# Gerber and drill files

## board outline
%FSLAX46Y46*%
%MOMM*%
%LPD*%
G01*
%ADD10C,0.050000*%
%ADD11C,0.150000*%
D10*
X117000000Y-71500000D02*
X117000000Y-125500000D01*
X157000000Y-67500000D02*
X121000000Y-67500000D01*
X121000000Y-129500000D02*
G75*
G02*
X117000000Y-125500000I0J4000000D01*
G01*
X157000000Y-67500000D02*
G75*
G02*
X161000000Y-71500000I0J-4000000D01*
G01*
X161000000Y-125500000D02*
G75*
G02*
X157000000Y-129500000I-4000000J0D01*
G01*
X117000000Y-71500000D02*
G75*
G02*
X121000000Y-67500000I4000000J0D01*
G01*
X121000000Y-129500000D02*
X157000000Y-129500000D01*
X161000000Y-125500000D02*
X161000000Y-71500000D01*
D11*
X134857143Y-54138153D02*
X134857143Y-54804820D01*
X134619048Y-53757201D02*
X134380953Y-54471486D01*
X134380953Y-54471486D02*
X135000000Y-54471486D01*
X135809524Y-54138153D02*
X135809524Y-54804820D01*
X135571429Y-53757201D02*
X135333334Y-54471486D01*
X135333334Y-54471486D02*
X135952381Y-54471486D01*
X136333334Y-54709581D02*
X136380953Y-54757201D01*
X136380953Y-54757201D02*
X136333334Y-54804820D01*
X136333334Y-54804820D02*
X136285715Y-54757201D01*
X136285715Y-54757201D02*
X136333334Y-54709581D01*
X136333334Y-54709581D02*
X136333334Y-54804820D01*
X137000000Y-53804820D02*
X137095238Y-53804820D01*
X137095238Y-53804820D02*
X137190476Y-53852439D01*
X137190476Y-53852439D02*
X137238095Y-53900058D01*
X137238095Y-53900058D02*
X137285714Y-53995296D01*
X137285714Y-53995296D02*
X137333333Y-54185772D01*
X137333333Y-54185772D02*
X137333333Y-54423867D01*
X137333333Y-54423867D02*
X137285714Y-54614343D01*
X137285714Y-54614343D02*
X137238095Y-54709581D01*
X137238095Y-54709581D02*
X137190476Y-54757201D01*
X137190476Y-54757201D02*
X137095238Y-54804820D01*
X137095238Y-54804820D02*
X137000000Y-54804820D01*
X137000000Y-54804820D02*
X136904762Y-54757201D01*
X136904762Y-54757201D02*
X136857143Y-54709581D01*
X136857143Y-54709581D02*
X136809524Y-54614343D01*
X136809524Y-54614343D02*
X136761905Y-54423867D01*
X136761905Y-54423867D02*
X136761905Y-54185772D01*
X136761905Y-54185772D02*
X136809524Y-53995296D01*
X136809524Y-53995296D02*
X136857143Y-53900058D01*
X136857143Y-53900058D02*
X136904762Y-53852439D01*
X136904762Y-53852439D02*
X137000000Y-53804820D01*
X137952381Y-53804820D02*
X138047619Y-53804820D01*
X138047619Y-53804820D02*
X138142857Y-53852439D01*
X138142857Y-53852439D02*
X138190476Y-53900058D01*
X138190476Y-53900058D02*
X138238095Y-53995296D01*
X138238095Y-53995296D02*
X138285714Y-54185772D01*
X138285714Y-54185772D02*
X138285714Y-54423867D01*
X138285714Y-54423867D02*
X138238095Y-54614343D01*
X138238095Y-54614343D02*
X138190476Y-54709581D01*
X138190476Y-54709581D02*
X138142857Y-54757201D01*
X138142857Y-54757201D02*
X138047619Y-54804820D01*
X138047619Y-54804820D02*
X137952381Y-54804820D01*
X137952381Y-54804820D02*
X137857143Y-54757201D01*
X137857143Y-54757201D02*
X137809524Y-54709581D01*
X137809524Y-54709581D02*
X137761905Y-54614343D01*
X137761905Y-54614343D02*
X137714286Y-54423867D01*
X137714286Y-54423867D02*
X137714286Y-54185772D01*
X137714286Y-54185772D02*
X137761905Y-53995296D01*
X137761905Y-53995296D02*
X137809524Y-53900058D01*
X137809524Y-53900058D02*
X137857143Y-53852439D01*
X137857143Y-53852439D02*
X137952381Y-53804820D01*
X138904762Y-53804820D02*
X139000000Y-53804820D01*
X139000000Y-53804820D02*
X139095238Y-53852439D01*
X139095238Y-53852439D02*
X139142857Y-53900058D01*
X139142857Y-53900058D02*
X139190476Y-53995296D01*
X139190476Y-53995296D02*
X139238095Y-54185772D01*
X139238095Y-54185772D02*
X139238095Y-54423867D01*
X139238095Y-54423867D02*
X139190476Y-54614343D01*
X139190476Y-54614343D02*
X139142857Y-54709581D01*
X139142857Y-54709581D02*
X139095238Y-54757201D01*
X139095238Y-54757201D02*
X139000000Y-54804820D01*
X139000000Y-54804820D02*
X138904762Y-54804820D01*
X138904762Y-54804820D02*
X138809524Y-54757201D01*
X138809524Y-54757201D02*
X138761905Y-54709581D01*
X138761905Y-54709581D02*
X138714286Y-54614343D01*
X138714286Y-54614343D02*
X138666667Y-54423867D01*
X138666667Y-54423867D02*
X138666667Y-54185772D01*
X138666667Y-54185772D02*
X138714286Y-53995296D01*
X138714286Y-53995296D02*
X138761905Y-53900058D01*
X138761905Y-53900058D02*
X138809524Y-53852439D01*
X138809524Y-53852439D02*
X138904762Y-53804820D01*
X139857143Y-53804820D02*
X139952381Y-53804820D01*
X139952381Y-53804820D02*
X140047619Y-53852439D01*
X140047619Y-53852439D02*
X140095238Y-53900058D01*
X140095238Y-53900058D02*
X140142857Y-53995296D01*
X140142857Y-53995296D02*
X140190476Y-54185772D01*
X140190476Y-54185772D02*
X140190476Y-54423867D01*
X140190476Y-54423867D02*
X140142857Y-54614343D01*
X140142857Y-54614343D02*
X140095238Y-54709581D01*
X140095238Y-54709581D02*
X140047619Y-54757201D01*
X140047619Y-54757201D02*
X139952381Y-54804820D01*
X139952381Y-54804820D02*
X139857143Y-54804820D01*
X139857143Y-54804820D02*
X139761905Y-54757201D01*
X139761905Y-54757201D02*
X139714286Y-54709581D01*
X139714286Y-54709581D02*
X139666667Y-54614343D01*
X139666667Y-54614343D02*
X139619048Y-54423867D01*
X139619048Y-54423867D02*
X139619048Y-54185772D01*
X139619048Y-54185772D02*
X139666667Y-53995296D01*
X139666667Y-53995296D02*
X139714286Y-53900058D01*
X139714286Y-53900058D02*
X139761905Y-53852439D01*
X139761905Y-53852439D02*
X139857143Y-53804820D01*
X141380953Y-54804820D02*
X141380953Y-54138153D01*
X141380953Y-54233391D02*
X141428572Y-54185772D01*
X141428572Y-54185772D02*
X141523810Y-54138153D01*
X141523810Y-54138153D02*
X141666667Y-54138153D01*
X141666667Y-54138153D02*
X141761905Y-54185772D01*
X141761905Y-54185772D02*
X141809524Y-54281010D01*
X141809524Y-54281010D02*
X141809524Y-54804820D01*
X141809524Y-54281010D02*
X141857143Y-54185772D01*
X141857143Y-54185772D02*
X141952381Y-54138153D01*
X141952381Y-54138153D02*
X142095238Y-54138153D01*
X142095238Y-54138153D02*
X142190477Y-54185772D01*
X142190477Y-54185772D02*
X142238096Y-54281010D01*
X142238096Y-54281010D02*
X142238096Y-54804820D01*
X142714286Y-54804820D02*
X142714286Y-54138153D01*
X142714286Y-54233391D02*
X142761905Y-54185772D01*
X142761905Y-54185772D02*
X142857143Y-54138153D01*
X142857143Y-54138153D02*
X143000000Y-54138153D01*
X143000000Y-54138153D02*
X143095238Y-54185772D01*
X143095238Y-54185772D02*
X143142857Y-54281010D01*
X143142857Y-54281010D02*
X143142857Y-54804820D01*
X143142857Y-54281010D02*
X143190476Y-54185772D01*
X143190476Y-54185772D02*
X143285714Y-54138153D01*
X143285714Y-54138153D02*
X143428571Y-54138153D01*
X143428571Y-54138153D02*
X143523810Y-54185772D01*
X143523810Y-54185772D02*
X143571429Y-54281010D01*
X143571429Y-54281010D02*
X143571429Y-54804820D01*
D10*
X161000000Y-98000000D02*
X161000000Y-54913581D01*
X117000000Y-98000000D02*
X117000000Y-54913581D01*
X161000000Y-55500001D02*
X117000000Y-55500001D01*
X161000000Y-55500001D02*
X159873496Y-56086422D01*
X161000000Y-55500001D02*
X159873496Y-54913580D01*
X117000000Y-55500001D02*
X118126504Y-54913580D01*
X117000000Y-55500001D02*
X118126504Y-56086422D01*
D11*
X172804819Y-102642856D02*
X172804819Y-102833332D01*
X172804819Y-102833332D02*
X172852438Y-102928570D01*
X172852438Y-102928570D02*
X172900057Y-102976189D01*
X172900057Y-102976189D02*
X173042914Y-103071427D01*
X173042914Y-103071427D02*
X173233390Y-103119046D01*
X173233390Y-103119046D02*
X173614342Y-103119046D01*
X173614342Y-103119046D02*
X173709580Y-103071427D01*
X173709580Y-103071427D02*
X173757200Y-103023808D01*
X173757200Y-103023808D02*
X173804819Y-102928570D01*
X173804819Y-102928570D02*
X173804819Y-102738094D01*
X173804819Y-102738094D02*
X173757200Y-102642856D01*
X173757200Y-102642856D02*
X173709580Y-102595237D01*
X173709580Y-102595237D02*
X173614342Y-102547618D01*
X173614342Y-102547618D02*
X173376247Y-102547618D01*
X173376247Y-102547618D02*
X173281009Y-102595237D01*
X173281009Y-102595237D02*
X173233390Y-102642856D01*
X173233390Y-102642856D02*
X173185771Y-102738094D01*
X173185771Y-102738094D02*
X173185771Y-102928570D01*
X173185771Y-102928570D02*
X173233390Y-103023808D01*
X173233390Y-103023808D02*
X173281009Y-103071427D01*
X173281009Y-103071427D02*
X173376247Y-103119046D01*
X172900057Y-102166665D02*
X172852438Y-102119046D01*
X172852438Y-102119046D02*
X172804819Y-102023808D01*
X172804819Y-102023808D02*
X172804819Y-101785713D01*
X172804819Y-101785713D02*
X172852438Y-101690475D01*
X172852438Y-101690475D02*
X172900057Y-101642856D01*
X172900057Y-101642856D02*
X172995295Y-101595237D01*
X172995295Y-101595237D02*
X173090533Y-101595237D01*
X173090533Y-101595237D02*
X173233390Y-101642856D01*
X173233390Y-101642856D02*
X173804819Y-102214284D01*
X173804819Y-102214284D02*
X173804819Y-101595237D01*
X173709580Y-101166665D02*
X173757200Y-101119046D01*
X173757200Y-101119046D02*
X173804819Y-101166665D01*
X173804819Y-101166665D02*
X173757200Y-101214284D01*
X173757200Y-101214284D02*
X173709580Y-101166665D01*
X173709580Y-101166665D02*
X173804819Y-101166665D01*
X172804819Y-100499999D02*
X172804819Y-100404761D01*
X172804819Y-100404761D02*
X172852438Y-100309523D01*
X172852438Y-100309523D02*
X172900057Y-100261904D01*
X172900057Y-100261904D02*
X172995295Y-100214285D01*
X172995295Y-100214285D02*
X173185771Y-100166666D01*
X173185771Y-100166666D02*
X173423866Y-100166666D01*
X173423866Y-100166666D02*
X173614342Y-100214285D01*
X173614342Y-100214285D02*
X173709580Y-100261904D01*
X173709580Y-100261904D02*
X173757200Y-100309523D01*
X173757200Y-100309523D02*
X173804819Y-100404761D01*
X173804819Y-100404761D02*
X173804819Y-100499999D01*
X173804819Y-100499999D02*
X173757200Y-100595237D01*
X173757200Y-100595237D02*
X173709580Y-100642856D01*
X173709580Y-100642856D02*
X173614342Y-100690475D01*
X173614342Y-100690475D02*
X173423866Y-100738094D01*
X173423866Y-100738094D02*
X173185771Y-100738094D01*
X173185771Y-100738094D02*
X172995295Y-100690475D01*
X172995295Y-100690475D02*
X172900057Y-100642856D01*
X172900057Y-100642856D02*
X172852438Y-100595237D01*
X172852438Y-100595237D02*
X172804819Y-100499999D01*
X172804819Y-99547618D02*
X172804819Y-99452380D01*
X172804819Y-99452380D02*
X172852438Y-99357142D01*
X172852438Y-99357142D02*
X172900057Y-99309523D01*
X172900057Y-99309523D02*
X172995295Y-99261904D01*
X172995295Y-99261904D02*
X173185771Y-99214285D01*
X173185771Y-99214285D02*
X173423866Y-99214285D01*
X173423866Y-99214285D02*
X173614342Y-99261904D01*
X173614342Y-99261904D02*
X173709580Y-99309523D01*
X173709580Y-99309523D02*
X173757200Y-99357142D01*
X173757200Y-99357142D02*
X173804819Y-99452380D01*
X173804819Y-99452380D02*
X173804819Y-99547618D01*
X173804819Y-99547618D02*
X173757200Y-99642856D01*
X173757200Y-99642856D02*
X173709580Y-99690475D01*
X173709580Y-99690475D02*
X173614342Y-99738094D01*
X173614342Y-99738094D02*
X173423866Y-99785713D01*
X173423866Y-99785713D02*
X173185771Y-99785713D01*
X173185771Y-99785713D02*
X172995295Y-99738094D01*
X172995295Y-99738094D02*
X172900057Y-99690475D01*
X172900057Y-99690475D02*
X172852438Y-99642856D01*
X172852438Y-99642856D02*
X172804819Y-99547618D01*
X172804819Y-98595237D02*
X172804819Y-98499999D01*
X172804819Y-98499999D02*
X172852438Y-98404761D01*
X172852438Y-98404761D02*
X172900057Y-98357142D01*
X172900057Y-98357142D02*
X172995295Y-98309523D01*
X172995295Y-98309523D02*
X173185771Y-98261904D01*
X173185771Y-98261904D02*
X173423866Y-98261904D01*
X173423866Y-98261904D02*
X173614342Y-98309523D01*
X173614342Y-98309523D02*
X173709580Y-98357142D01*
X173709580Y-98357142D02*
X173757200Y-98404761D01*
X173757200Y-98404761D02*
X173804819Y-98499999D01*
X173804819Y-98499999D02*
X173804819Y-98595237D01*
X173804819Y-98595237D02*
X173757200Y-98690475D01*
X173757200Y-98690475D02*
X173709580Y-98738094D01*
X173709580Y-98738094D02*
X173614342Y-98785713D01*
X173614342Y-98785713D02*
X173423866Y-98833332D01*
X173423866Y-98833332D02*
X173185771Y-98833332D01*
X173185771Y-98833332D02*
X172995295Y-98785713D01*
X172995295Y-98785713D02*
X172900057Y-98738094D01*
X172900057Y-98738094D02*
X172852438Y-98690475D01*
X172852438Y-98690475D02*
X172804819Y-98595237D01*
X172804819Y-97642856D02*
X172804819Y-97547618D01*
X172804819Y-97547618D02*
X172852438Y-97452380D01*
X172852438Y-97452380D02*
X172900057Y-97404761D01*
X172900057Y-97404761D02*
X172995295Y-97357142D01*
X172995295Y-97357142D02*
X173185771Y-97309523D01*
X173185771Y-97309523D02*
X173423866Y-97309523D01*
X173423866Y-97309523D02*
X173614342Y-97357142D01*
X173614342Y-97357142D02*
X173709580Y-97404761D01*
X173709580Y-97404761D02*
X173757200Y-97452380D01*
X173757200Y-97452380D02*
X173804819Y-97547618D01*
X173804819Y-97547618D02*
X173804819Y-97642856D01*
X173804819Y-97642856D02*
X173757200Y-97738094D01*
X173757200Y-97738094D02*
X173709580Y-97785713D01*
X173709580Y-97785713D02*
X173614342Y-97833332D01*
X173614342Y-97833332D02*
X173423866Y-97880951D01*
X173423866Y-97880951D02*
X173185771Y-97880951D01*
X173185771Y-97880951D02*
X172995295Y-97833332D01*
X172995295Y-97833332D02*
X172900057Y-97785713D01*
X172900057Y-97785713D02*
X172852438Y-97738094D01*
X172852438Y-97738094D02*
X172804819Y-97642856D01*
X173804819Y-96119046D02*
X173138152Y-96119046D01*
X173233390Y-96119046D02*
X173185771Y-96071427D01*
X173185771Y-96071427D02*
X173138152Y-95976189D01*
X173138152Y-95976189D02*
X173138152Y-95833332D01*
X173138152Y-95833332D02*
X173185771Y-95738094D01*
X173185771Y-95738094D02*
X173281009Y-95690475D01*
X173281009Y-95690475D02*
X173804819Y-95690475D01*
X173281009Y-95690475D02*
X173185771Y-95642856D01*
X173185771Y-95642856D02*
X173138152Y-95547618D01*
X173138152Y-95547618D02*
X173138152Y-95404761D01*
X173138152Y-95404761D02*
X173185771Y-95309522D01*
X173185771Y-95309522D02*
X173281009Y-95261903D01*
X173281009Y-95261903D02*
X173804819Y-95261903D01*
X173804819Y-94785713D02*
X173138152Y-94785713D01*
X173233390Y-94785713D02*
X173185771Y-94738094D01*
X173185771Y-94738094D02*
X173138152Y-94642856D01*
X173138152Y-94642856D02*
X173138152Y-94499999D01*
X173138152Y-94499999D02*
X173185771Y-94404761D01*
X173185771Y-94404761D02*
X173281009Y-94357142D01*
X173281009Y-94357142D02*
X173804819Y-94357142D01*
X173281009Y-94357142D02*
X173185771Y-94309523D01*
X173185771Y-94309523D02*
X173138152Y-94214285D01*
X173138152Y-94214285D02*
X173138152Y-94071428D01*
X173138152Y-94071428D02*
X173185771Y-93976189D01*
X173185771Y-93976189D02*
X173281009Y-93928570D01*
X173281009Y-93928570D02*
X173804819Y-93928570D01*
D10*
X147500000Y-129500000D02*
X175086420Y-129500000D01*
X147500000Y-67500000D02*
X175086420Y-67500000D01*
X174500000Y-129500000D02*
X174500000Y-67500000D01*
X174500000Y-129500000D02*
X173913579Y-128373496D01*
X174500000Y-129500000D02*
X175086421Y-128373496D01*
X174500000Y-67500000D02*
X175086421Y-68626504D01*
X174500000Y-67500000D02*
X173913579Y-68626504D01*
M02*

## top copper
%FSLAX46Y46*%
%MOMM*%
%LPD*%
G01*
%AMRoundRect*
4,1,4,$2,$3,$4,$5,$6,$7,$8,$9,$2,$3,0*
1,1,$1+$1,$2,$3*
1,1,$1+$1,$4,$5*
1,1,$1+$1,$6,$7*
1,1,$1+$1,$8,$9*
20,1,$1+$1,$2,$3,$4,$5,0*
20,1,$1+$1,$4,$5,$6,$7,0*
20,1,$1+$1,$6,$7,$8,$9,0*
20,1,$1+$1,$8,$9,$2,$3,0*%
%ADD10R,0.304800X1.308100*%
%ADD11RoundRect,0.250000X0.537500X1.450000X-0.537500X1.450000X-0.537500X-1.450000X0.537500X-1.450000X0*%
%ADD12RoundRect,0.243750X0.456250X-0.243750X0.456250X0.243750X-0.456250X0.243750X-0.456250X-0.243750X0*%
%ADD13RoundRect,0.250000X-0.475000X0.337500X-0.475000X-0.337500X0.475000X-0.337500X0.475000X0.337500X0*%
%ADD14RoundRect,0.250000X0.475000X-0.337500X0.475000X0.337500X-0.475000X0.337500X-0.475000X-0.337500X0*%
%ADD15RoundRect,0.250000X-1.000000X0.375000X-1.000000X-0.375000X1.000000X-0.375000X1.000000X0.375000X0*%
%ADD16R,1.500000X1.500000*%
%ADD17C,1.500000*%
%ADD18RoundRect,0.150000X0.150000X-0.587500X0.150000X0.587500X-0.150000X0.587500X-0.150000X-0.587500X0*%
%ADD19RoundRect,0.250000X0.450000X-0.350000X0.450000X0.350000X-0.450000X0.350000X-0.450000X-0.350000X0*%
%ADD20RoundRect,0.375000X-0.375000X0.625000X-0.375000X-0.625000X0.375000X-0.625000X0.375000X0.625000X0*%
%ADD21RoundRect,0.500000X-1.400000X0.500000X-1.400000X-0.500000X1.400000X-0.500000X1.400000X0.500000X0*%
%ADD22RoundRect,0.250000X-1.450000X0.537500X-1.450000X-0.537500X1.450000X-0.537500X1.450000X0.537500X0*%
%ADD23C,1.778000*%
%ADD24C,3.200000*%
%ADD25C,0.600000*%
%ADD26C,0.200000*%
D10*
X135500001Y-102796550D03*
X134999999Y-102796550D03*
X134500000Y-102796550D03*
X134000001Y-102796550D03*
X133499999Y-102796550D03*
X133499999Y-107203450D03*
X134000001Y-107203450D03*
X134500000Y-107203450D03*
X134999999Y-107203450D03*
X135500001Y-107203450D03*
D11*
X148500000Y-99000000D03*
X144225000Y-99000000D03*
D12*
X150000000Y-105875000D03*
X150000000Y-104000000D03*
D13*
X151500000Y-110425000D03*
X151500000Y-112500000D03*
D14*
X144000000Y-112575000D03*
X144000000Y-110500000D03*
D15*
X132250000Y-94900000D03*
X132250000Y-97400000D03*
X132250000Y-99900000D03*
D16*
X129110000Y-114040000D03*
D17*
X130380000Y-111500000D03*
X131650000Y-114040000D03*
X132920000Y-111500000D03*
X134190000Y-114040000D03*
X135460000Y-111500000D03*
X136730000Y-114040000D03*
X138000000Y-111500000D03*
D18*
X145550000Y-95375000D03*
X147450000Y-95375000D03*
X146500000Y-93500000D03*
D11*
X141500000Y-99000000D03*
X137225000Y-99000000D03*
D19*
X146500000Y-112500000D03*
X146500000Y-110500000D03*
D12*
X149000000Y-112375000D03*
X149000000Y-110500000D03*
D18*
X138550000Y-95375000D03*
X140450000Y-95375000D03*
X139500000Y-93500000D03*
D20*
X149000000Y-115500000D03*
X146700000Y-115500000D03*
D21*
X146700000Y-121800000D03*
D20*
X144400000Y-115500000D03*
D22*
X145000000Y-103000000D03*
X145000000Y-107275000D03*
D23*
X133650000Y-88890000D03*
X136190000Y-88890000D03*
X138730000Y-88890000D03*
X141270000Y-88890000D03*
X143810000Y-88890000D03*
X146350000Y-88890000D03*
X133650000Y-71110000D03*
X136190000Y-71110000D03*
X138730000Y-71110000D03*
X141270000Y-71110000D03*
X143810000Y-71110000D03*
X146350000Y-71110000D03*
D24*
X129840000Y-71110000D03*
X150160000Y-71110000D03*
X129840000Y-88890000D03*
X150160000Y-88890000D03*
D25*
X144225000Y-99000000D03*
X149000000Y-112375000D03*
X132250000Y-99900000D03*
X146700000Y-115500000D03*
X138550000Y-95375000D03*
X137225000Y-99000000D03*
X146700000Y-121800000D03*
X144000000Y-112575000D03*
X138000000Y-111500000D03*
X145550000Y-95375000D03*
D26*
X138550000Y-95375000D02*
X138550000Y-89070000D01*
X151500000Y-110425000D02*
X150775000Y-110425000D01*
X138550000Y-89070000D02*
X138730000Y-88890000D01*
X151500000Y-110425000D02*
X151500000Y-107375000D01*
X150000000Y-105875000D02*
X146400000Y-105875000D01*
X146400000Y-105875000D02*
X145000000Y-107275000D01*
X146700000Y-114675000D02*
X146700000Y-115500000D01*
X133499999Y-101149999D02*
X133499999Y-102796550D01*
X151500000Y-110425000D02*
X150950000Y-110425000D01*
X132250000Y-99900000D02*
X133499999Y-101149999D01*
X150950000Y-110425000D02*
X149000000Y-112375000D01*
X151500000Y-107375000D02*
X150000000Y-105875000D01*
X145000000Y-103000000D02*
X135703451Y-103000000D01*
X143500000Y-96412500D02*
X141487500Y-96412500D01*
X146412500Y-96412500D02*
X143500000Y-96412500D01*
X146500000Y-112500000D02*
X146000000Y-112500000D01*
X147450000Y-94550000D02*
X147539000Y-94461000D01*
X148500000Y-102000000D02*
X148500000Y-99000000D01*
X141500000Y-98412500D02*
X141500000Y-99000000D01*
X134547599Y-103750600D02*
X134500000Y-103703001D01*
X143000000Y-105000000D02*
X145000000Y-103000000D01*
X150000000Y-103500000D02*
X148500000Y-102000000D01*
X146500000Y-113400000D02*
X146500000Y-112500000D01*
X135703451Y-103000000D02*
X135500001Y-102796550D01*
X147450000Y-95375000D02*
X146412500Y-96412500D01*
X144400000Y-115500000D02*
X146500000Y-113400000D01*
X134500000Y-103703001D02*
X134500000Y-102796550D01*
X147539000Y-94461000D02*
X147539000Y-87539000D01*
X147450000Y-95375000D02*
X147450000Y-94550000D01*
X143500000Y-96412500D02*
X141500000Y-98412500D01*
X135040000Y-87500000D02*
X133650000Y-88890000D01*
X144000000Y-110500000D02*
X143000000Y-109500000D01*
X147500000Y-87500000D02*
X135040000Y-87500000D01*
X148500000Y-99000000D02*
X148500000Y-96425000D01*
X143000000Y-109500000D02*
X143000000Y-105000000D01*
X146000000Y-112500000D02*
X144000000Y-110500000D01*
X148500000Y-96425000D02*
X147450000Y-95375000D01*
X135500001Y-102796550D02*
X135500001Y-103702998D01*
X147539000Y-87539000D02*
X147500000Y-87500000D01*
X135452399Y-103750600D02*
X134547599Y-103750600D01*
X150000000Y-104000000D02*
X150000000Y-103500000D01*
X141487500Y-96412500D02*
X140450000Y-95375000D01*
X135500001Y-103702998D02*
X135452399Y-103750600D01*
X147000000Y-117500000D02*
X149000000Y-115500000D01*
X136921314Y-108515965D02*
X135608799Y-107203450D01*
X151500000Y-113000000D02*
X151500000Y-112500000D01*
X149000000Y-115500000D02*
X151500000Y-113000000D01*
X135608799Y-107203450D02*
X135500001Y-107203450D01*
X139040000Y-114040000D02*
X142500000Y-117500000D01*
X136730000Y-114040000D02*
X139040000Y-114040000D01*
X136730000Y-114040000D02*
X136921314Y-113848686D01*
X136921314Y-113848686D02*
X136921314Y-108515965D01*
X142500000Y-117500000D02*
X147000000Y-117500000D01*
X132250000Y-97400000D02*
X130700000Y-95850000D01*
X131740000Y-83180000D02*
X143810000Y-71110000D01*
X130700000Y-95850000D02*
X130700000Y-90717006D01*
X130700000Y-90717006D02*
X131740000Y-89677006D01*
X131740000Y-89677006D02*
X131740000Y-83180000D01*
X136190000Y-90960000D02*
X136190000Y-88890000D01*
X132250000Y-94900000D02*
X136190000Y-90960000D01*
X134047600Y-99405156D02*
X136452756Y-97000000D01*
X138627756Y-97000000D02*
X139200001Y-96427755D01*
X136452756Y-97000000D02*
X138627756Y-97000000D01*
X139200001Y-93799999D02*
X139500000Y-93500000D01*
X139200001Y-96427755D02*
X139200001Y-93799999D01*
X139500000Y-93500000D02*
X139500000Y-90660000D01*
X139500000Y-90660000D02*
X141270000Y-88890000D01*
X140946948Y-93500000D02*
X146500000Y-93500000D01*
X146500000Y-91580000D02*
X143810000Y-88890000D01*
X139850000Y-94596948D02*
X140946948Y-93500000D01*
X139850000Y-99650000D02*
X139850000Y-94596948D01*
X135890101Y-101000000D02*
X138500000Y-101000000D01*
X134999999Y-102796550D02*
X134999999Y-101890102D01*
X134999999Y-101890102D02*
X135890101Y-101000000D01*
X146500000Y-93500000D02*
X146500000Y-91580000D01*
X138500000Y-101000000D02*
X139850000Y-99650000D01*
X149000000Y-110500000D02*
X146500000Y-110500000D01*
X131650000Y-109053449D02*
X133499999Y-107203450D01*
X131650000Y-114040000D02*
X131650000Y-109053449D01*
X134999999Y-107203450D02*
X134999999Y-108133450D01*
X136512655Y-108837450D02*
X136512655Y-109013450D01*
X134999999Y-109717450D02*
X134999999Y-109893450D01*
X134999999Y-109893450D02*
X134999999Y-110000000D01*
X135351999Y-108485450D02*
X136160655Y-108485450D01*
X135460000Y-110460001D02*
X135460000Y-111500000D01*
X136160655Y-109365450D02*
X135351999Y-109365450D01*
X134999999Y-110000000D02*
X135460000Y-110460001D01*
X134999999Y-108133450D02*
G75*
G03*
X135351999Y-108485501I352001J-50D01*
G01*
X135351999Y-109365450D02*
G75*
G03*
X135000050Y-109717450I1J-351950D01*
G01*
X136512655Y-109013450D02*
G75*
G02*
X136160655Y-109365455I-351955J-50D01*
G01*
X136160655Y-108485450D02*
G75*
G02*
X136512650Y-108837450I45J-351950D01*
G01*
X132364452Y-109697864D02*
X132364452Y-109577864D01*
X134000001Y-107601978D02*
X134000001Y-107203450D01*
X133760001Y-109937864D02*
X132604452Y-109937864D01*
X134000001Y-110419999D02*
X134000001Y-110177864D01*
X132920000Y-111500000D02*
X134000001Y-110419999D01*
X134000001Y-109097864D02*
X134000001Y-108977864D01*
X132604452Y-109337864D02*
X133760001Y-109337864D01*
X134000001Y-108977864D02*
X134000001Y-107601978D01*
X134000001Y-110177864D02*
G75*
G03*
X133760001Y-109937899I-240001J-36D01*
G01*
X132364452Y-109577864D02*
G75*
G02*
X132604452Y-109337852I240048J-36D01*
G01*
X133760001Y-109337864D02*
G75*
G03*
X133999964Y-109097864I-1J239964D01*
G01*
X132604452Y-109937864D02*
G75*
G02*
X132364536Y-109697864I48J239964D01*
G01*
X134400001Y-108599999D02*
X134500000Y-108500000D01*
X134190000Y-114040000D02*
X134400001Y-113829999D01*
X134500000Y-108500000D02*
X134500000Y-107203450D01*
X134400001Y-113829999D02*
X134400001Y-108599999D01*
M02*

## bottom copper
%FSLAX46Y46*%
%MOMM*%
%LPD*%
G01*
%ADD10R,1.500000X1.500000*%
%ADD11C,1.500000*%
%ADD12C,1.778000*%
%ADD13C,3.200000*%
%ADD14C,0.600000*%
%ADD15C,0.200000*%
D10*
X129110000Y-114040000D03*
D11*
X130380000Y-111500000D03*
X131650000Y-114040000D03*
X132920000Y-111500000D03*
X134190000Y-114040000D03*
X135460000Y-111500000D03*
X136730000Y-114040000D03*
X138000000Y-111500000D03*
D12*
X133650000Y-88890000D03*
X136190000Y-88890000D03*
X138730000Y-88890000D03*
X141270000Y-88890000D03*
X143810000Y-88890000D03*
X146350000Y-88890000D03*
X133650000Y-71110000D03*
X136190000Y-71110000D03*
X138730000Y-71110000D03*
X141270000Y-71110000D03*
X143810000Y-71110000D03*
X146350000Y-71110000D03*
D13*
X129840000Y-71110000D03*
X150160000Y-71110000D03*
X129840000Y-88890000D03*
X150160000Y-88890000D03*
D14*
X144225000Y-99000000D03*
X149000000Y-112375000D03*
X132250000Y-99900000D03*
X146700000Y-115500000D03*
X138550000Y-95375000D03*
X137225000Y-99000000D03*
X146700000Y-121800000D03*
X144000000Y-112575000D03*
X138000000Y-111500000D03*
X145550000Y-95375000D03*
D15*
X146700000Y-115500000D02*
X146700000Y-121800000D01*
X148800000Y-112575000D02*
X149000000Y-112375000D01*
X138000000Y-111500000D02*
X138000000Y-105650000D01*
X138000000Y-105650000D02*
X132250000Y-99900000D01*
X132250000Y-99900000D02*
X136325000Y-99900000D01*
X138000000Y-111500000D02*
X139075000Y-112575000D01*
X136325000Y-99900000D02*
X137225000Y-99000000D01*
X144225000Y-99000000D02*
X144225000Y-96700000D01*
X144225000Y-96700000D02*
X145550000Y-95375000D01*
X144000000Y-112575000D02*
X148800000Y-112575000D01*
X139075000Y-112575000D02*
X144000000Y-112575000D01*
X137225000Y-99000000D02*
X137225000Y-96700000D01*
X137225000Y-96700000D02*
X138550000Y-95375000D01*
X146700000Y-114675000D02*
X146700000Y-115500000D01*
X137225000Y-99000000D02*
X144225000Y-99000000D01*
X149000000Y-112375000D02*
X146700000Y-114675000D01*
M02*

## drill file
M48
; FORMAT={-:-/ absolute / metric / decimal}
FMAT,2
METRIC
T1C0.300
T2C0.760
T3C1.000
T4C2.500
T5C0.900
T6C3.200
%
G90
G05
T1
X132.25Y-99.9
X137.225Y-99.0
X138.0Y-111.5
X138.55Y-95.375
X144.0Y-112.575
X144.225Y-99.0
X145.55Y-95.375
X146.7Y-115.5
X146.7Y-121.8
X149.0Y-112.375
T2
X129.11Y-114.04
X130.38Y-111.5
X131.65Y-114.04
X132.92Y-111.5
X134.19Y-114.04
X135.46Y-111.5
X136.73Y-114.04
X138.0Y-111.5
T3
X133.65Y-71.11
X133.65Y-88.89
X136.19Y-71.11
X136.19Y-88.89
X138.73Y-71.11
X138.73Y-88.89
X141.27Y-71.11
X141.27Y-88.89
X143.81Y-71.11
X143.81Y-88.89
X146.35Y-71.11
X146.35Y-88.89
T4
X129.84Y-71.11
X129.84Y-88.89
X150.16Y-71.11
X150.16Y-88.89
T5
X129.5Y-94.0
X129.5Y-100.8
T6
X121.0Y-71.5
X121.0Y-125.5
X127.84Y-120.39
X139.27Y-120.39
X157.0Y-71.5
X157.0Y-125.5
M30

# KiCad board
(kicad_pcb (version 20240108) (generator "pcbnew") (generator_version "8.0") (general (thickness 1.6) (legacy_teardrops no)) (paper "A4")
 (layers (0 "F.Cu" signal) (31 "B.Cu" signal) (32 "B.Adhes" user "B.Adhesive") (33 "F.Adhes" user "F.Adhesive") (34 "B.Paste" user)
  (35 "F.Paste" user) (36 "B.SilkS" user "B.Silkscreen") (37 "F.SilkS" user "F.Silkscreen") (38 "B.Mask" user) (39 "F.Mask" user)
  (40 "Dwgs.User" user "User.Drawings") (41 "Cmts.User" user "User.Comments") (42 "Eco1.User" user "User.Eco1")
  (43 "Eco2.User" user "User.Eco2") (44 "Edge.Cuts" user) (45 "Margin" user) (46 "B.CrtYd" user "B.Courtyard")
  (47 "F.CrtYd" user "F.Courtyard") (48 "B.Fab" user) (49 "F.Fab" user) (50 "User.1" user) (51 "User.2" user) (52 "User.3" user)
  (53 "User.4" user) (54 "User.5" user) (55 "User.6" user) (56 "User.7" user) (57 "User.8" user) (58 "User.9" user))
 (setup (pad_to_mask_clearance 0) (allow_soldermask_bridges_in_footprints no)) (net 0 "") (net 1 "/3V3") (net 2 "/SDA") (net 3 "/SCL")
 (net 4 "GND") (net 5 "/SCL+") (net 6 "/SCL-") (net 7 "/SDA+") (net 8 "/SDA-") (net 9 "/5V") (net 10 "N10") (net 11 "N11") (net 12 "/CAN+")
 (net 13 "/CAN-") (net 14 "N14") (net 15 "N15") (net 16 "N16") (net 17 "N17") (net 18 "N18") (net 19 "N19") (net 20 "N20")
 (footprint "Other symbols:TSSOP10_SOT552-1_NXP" (layer "F.Cu") (at 134.5 105 -90)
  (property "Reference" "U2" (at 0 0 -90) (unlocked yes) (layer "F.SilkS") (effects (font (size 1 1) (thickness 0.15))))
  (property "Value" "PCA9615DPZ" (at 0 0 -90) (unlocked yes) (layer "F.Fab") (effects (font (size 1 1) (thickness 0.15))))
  (pad "1" smd rect (at -2.20345 -1.000001 270) (size 1.3081 0.3048) (layers "F.Cu" "F.Paste" "F.Mask") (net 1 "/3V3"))
  (pad "2" smd rect (at -2.20345 -0.499999 270) (size 1.3081 0.3048) (layers "F.Cu" "F.Paste" "F.Mask") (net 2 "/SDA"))
  (pad "3" smd rect (at -2.20345 0 270) (size 1.3081 0.3048) (layers "F.Cu" "F.Paste" "F.Mask") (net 1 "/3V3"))
  (pad "4" smd rect (at -2.20345 0.499999 270) (size 1.3081 0.3048) (layers "F.Cu" "F.Paste" "F.Mask") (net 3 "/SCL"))
  (pad "5" smd rect (at -2.20345 1.000001 270) (size 1.3081 0.3048) (layers "F.Cu" "F.Paste" "F.Mask") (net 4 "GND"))
  (pad "6" smd rect (at 2.20345 1.000001 270) (size 1.3081 0.3048) (layers "F.Cu" "F.Paste" "F.Mask") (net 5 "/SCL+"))
  (pad "7" smd rect (at 2.20345 0.499999 270) (size 1.3081 0.3048) (layers "F.Cu" "F.Paste" "F.Mask") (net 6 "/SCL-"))
  (pad "8" smd rect (at 2.20345 0 270) (size 1.3081 0.3048) (layers "F.Cu" "F.Paste" "F.Mask") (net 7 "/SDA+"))
  (pad "9" smd rect (at 2.20345 -0.499999 270) (size 1.3081 0.3048) (layers "F.Cu" "F.Paste" "F.Mask") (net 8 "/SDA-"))
  (pad "10" smd rect (at 2.20345 -1.000001 270) (size 1.3081 0.3048) (layers "F.Cu" "F.Paste" "F.Mask") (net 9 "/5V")))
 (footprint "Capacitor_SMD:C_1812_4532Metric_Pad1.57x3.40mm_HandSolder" (layer "F.Cu") (at 146.3625 99 180)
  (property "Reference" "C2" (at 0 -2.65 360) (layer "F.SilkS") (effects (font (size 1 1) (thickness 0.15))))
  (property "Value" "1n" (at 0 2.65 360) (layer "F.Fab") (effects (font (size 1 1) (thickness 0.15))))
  (pad "1" smd roundrect (at -2.1375 0 180) (size 1.575 3.4) (layers "F.Cu" "F.Paste" "F.Mask") (roundrect_rratio 0.15873) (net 1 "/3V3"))
  (pad "2" smd roundrect (at 2.1375 0 180) (size 1.575 3.4) (layers "F.Cu" "F.Paste" "F.Mask") (roundrect_rratio 0.15873) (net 4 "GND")))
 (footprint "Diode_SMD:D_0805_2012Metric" (layer "F.Cu") (at 150 104.9375 90)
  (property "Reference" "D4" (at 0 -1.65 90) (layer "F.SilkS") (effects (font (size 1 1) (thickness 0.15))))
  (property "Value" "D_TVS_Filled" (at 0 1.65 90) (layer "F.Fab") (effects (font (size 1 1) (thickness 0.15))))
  (pad "1" smd roundrect (at -0.9375 0 90) (size 0.975 1.4) (layers "F.Cu" "F.Paste" "F.Mask") (roundrect_rratio 0.25) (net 4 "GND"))
  (pad "2" smd roundrect (at 0.9375 0 90) (size 0.975 1.4) (layers "F.Cu" "F.Paste" "F.Mask") (roundrect_rratio 0.25) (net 1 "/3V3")))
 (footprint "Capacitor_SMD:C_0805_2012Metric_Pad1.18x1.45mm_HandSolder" (layer "F.Cu") (at 151.5 111.4625 -90)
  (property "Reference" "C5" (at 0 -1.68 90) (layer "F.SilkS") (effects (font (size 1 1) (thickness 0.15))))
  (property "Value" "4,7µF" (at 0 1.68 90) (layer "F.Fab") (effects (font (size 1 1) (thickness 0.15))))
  (pad "1" smd roundrect (at -1.0375 0 270) (size 1.175 1.45) (layers "F.Cu" "F.Paste" "F.Mask") (roundrect_rratio 0.212766) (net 4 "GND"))
  (pad "2" smd roundrect (at 1.0375 0 270) (size 1.175 1.45) (layers "F.Cu" "F.Paste" "F.Mask") (roundrect_rratio 0.212766) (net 9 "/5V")))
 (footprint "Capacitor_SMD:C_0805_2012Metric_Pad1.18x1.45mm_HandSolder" (layer "F.Cu") (at 144 111.5375 90)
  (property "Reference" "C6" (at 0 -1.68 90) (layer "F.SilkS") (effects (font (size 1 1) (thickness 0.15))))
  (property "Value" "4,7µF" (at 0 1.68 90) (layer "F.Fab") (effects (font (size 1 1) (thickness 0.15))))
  (pad "1" smd roundrect (at -1.0375 0 90) (size 1.175 1.45) (layers "F.Cu" "F.Paste" "F.Mask") (roundrect_rratio 0.212766) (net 4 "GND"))
  (pad "2" smd roundrect (at 1.0375 0 90) (size 1.175 1.45) (layers "F.Cu" "F.Paste" "F.Mask") (roundrect_rratio 0.212766) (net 1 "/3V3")))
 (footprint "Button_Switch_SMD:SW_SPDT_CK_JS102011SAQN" (layer "F.Cu") (at 129.5 97.4 -90)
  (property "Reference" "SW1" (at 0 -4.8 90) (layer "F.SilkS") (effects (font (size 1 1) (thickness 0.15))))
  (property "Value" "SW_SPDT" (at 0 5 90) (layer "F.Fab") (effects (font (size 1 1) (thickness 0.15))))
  (pad "" np_thru_hole circle (at -3.4 0 270) (size 0.9 0.9) (drill 0.9) (layers "*.Cu" "*.Mask"))
  (pad "" np_thru_hole circle (at 3.4 0 270) (size 0.9 0.9) (drill 0.9) (layers "*.Cu" "*.Mask"))
  (pad "1" smd roundrect (at -2.5 -2.75 270) (size 1.25 2.5) (layers "F.Cu" "F.Paste" "F.Mask") (roundrect_rratio 0.2) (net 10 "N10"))
  (pad "2" smd roundrect (at 0 -2.75 270) (size 1.25 2.5) (layers "F.Cu" "F.Paste" "F.Mask") (roundrect_rratio 0.2) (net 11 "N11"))
  (pad "3" smd roundrect (at 2.5 -2.75 270) (size 1.25 2.5) (layers "F.Cu" "F.Paste" "F.Mask") (roundrect_rratio 0.2) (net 4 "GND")))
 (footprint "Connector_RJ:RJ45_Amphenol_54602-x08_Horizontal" (layer "F.Cu") (at 129.11 114.04)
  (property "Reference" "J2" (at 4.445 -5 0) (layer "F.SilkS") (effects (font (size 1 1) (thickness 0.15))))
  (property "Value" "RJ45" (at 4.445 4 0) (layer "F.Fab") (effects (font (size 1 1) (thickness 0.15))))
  (pad "" np_thru_hole circle (at -1.27 6.35) (size 3.2 3.2) (drill 3.2) (layers "*.Cu" "*.Mask"))
  (pad "" np_thru_hole circle (at 10.16 6.35) (size 3.2 3.2) (drill 3.2) (layers "*.Cu" "*.Mask"))
  (pad "1" thru_hole rect (at 0 0) (size 1.5 1.5) (drill 0.76) (layers "*.Cu" "*.Mask") (remove_unused_layers no) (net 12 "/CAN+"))
  (pad "2" thru_hole circle (at 1.27 -2.54) (size 1.5 1.5) (drill 0.76) (layers "*.Cu" "*.Mask") (remove_unused_layers no) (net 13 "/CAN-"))
  (pad "3" thru_hole circle (at 2.54 0) (size 1.5 1.5) (drill 0.76) (layers "*.Cu" "*.Mask") (remove_unused_layers no) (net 5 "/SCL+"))
  (pad "4" thru_hole circle (at 3.81 -2.54) (size 1.5 1.5) (drill 0.76) (layers "*.Cu" "*.Mask") (remove_unused_layers no) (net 6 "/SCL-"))
  (pad "5" thru_hole circle (at 5.08 0) (size 1.5 1.5) (drill 0.76) (layers "*.Cu" "*.Mask") (remove_unused_layers no) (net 7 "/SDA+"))
  (pad "6" thru_hole circle (at 6.35 -2.54) (size 1.5 1.5) (drill 0.76) (layers "*.Cu" "*.Mask") (remove_unused_layers no) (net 8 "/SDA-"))
  (pad "7" thru_hole circle (at 7.62 0) (size 1.5 1.5) (drill 0.76) (layers "*.Cu" "*.Mask") (remove_unused_layers no) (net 9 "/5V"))
  (pad "8" thru_hole circle (at 8.89 -2.54) (size 1.5 1.5) (drill 0.76) (layers "*.Cu" "*.Mask") (remove_unused_layers no) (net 4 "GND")))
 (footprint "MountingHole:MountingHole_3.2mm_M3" (layer "F.Cu") (at 121 71.5)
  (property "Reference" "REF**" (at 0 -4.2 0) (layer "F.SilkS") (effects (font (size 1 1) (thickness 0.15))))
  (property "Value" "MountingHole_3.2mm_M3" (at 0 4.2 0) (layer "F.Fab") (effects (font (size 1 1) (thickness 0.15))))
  (pad "" np_thru_hole circle (at 0 0) (size 3.2 3.2) (drill 3.2) (layers "*.Cu" "*.Mask")))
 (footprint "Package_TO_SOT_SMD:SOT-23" (layer "F.Cu") (at 146.5 94.4375 90)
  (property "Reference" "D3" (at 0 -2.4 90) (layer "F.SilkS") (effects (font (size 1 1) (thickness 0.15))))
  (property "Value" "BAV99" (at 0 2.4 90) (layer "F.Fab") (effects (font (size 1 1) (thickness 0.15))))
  (pad "1" smd roundrect (at -0.9375 -0.95 90) (size 1.475 0.6) (layers "F.Cu" "F.Paste" "F.Mask") (roundrect_rratio 0.25) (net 4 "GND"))
  (pad "2" smd roundrect (at -0.9375 0.95 90) (size 1.475 0.6) (layers "F.Cu" "F.Paste" "F.Mask") (roundrect_rratio 0.25) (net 1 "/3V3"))
  (pad "3" smd roundrect (at 0.9375 0 90) (size 1.475 0.6) (layers "F.Cu" "F.Paste" "F.Mask") (roundrect_rratio 0.25) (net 2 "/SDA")))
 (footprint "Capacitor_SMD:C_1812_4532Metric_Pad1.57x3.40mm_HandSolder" (layer "F.Cu") (at 139.3625 99 180)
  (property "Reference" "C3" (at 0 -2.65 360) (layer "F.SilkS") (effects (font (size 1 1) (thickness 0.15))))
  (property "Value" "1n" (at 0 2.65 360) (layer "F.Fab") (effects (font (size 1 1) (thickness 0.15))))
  (pad "1" smd roundrect (at -2.1375 0 180) (size 1.575 3.4) (layers "F.Cu" "F.Paste" "F.Mask") (roundrect_rratio 0.15873) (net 1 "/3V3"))
  (pad "2" smd roundrect (at 2.1375 0 180) (size 1.575 3.4) (layers "F.Cu" "F.Paste" "F.Mask") (roundrect_rratio 0.15873) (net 4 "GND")))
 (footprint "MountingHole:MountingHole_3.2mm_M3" (layer "F.Cu") (at 157 125.5)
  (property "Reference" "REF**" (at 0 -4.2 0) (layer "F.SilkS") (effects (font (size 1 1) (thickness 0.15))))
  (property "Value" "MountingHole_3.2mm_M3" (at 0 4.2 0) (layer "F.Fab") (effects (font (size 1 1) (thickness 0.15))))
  (pad "" np_thru_hole circle (at 0 0) (size 3.2 3.2) (drill 3.2) (layers "*.Cu" "*.Mask")))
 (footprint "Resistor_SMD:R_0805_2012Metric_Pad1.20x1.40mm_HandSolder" (layer "F.Cu") (at 146.5 111.5 90)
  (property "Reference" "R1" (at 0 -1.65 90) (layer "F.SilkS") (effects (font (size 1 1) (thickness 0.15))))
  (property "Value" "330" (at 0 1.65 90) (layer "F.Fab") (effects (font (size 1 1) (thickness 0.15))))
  (pad "1" smd roundrect (at -1 0 90) (size 1.2 1.4) (layers "F.Cu" "F.Paste" "F.Mask") (roundrect_rratio 0.208333) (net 1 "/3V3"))
  (pad "2" smd roundrect (at 1 0 90) (size 1.2 1.4) (layers "F.Cu" "F.Paste" "F.Mask") (roundrect_rratio 0.208333) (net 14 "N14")))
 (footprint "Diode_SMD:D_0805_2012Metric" (layer "F.Cu") (at 149 111.4375 90)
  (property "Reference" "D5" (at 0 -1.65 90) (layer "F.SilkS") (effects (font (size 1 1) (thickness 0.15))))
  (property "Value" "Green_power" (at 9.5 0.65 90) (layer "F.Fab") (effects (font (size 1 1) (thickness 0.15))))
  (pad "1" smd roundrect (at -0.9375 0 90) (size 0.975 1.4) (layers "F.Cu" "F.Paste" "F.Mask") (roundrect_rratio 0.25) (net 4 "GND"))
  (pad "2" smd roundrect (at 0.9375 0 90) (size 0.975 1.4) (layers "F.Cu" "F.Paste" "F.Mask") (roundrect_rratio 0.25) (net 14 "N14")))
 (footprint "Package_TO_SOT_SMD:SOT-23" (layer "F.Cu") (at 139.5 94.4375 90)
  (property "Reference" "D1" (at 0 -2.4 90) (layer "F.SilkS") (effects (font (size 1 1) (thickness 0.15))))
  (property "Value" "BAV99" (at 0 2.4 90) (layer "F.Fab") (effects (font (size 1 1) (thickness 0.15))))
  (pad "1" smd roundrect (at -0.9375 -0.95 90) (size 1.475 0.6) (layers "F.Cu" "F.Paste" "F.Mask") (roundrect_rratio 0.25) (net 4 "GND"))
  (pad "2" smd roundrect (at -0.9375 0.95 90) (size 1.475 0.6) (layers "F.Cu" "F.Paste" "F.Mask") (roundrect_rratio 0.25) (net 1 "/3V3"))
  (pad "3" smd roundrect (at 0.9375 0 90) (size 1.475 0.6) (layers "F.Cu" "F.Paste" "F.Mask") (roundrect_rratio 0.25) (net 3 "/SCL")))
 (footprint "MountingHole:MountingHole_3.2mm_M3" (layer "F.Cu") (at 121 125.5)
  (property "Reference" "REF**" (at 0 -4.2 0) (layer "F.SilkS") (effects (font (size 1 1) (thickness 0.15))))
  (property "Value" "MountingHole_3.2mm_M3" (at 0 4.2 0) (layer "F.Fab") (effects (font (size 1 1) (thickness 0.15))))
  (pad "" np_thru_hole circle (at 0 0) (size 3.2 3.2) (drill 3.2) (layers "*.Cu" "*.Mask")))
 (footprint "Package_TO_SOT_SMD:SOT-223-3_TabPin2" (layer "F.Cu") (at 146.7 118.65 -90)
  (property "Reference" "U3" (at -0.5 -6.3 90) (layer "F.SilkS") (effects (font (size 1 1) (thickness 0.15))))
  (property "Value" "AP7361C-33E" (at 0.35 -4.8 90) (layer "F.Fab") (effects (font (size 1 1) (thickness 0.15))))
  (pad "1" smd roundrect (at -3.15 -2.3 270) (size 2 1.5) (layers "F.Cu" "F.Paste" "F.Mask") (roundrect_rratio 0.25) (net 9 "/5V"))
  (pad "2" smd roundrect (at -3.15 0 270) (size 2 1.5) (layers "F.Cu" "F.Paste" "F.Mask") (roundrect_rratio 0.25) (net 4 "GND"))
  (pad "2" smd roundrect (at 3.15 0 270) (size 2 3.8) (layers "F.Cu" "F.Paste" "F.Mask") (roundrect_rratio 0.25) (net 4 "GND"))
  (pad "3" smd roundrect (at -3.15 2.3 270) (size 2 1.5) (layers "F.Cu" "F.Paste" "F.Mask") (roundrect_rratio 0.25) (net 1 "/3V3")))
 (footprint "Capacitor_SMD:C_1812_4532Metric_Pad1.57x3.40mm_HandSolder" (layer "F.Cu") (at 145 105.1375 -90)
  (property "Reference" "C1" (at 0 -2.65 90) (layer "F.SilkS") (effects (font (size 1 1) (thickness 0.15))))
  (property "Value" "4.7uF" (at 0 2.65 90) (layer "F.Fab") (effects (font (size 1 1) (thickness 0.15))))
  (pad "1" smd roundrect (at -2.1375 0 270) (size 1.575 3.4) (layers "F.Cu" "F.Paste" "F.Mask") (roundrect_rratio 0.15873) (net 1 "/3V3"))
  (pad "2" smd roundrect (at 2.1375 0 270) (size 1.575 3.4) (layers "F.Cu" "F.Paste" "F.Mask") (roundrect_rratio 0.15873) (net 4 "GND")))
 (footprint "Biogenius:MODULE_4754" (layer "F.Cu") (at 140 80)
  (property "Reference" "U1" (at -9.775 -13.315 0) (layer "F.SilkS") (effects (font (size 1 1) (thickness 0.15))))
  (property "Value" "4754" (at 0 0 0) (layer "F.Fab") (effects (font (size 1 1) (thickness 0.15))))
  (pad "JP1_1" thru_hole circle (at -6.35 8.89) (size 1.778 1.778) (drill 1) (layers "*.Cu" "*.Mask") (remove_unused_layers no)
   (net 1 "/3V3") (solder_mask_margin 0.102))
  (pad "JP1_2" thru_hole circle (at -3.81 8.89) (size 1.778 1.778) (drill 1) (layers "*.Cu" "*.Mask") (remove_unused_layers no)
   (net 10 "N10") (solder_mask_margin 0.102))
  (pad "JP1_3" thru_hole circle (at -1.27 8.89) (size 1.778 1.778) (drill 1) (layers "*.Cu" "*.Mask") (remove_unused_layers no)
   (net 4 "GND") (solder_mask_margin 0.102))
  (pad "JP1_4" thru_hole circle (at 1.27 8.89) (size 1.778 1.778) (drill 1) (layers "*.Cu" "*.Mask") (remove_unused_layers no)
   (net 3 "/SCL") (solder_mask_margin 0.102))
  (pad "JP1_5" thru_hole circle (at 3.81 8.89) (size 1.778 1.778) (drill 1) (layers "*.Cu" "*.Mask") (remove_unused_layers no)
   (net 2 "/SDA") (solder_mask_margin 0.102))
  (pad "JP1_6" thru_hole circle (at 6.35 8.89) (size 1.778 1.778) (drill 1) (layers "*.Cu" "*.Mask") (remove_unused_layers no)
   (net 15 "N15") (solder_mask_margin 0.102))
  (pad "JP2_1" thru_hole circle (at -6.35 -8.89) (size 1.778 1.778) (drill 1) (layers "*.Cu" "*.Mask") (remove_unused_layers no)
   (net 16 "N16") (solder_mask_margin 0.102))
  (pad "JP2_2" thru_hole circle (at -3.81 -8.89) (size 1.778 1.778) (drill 1) (layers "*.Cu" "*.Mask") (remove_unused_layers no)
   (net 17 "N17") (solder_mask_margin 0.102))
  (pad "JP2_3" thru_hole circle (at -1.27 -8.89) (size 1.778 1.778) (drill 1) (layers "*.Cu" "*.Mask") (remove_unused_layers no)
   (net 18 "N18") (solder_mask_margin 0.102))
  (pad "JP2_4" thru_hole circle (at 1.27 -8.89) (size 1.778 1.778) (drill 1) (layers "*.Cu" "*.Mask") (remove_unused_layers no)
   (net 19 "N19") (solder_mask_margin 0.102))
  (pad "JP2_5" thru_hole circle (at 3.81 -8.89) (size 1.778 1.778) (drill 1) (layers "*.Cu" "*.Mask") (remove_unused_layers no)
   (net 11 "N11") (solder_mask_margin 0.102))
  (pad "JP2_6" thru_hole circle (at 6.35 -8.89) (size 1.778 1.778) (drill 1) (layers "*.Cu" "*.Mask") (remove_unused_layers no)
   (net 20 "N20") (solder_mask_margin 0.102))
  (pad "P1" thru_hole circle (at -10.16 -8.89) (size 3.2 3.2) (drill 2.5) (layers "*.Cu" "*.Mask") (remove_unused_layers no)
   (solder_mask_margin 0.102))
  (pad "P2" thru_hole circle (at 10.16 -8.89) (size 3.2 3.2) (drill 2.5) (layers "*.Cu" "*.Mask") (remove_unused_layers no)
   (solder_mask_margin 0.102))
  (pad "P3" thru_hole circle (at -10.16 8.89) (size 3.2 3.2) (drill 2.5) (layers "*.Cu" "*.Mask") (remove_unused_layers no)
   (solder_mask_margin 0.102))
  (pad "P4" thru_hole circle (at 10.16 8.89) (size 3.2 3.2) (drill 2.5) (layers "*.Cu" "*.Mask") (remove_unused_layers no)
   (solder_mask_margin 0.102)))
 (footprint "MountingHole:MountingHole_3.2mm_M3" (layer "F.Cu") (at 157 71.5)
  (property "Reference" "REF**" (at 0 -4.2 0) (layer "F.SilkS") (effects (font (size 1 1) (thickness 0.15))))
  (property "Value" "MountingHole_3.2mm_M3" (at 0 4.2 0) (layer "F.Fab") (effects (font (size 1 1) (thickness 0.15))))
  (pad "" np_thru_hole circle (at 0 0) (size 3.2 3.2) (drill 3.2) (layers "*.Cu" "*.Mask")))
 (gr_line (start 117 71.5) (end 117 125.5) (stroke (width 0.05) (type default)) (layer "Edge.Cuts"))
 (gr_line (start 157 67.5) (end 121 67.5) (stroke (width 0.05) (type default)) (layer "Edge.Cuts"))
 (gr_arc (start 121 129.5) (mid 118.171573 128.328427) (end 117 125.5) (stroke (width 0.05) (type default)) (layer "Edge.Cuts"))
 (gr_arc (start 157 67.5) (mid 159.828427 68.671573) (end 161 71.5) (stroke (width 0.05) (type default)) (layer "Edge.Cuts"))
 (gr_arc (start 161 125.5) (mid 159.828427 128.328427) (end 157 129.5) (stroke (width 0.05) (type default)) (layer "Edge.Cuts"))
 (gr_arc (start 117 71.5) (mid 118.171573 68.671573) (end 121 67.5) (stroke (width 0.05) (type default)) (layer "Edge.Cuts"))
 (gr_line (start 121 129.5) (end 157 129.5) (stroke (width 0.05) (type default)) (layer "Edge.Cuts"))
 (gr_line (start 161 125.5) (end 161 71.5) (stroke (width 0.05) (type default)) (layer "Edge.Cuts"))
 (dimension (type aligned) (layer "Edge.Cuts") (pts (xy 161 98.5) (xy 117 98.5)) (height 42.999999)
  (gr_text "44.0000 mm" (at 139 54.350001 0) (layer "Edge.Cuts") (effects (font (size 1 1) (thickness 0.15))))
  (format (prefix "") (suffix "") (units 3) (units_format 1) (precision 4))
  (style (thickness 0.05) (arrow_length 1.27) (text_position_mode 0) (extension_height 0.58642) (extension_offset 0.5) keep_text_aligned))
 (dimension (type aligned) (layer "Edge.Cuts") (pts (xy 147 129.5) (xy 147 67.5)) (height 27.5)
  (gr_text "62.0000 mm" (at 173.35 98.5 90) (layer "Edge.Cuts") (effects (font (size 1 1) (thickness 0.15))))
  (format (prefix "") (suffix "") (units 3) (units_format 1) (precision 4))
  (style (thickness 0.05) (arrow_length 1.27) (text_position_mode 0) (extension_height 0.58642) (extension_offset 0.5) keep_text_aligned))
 (segment (start 138.55 95.375) (end 138.55 89.07) (width 0.2) (layer "F.Cu") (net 4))
 (segment (start 151.5 110.425) (end 150.775 110.425) (width 0.2) (layer "F.Cu") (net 4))
 (segment (start 138.55 89.07) (end 138.73 88.89) (width 0.2) (layer "F.Cu") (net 4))
 (segment (start 151.5 110.425) (end 151.5 107.375) (width 0.2) (layer "F.Cu") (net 4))
 (segment (start 150 105.875) (end 146.4 105.875) (width 0.2) (layer "F.Cu") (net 4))
 (segment (start 146.4 105.875) (end 145 107.275) (width 0.2) (layer "F.Cu") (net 4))
 (segment (start 146.7 114.675) (end 146.7 115.5) (width 0.2) (layer "F.Cu") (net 4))
 (segment (start 133.499999 101.149999) (end 133.499999 102.79655) (width 0.2) (layer "F.Cu") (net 4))
 (segment (start 151.5 110.425) (end 150.95 110.425) (width 0.2) (layer "F.Cu") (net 4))
 (segment (start 132.25 99.9) (end 133.499999 101.149999) (width 0.2) (layer "F.Cu") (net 4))
 (segment (start 150.95 110.425) (end 149 112.375) (width 0.2) (layer "F.Cu") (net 4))
 (segment (start 151.5 107.375) (end 150 105.875) (width 0.2) (layer "F.Cu") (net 4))
 (via (at 144.225 99) (size 0.6) (drill 0.3) (layers "F.Cu" "B.Cu") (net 4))
 (via (at 149 112.375) (size 0.6) (drill 0.3) (layers "F.Cu" "B.Cu") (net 4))
 (via (at 132.25 99.9) (size 0.6) (drill 0.3) (layers "F.Cu" "B.Cu") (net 4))
 (via (at 146.7 115.5) (size 0.6) (drill 0.3) (layers "F.Cu" "B.Cu") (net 4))
 (via (at 138.55 95.375) (size 0.6) (drill 0.3) (layers "F.Cu" "B.Cu") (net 4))
 (via (at 137.225 99) (size 0.6) (drill 0.3) (layers "F.Cu" "B.Cu") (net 4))
 (via (at 146.7 121.8) (size 0.6) (drill 0.3) (layers "F.Cu" "B.Cu") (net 4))
 (via (at 144 112.575) (size 0.6) (drill 0.3) (layers "F.Cu" "B.Cu") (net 4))
 (via (at 138 111.5) (size 0.6) (drill 0.3) (layers "F.Cu" "B.Cu") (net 4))
 (via (at 145.55 95.375) (size 0.6) (drill 0.3) (layers "F.Cu" "B.Cu") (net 4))
 (segment (start 146.7 115.5) (end 146.7 121.8) (width 0.2) (layer "B.Cu") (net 4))
 (segment (start 148.8 112.575) (end 149 112.375) (width 0.2) (layer "B.Cu") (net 4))
 (segment (start 138 111.5) (end 138 105.65) (width 0.2) (layer "B.Cu") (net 4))
 (segment (start 138 105.65) (end 132.25 99.9) (width 0.2) (layer "B.Cu") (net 4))
 (segment (start 132.25 99.9) (end 136.325 99.9) (width 0.2) (layer "B.Cu") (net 4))
 (segment (start 138 111.5) (end 139.075 112.575) (width 0.2) (layer "B.Cu") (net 4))
 (segment (start 136.325 99.9) (end 137.225 99) (width 0.2) (layer "B.Cu") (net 4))
 (segment (start 144.225 99) (end 144.225 96.7) (width 0.2) (layer "B.Cu") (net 4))
 (segment (start 144.225 96.7) (end 145.55 95.375) (width 0.2) (layer "B.Cu") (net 4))
 (segment (start 144 112.575) (end 148.8 112.575) (width 0.2) (layer "B.Cu") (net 4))
 (segment (start 139.075 112.575) (end 144 112.575) (width 0.2) (layer "B.Cu") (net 4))
 (segment (start 137.225 99) (end 137.225 96.7) (width 0.2) (layer "B.Cu") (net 4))
 (segment (start 137.225 96.7) (end 138.55 95.375) (width 0.2) (layer "B.Cu") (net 4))
 (segment (start 146.7 114.675) (end 146.7 115.5) (width 0.2) (layer "B.Cu") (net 4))
 (segment (start 137.225 99) (end 144.225 99) (width 0.2) (layer "B.Cu") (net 4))
 (segment (start 149 112.375) (end 146.7 114.675) (width 0.2) (layer "B.Cu") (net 4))
 (segment (start 145 103) (end 135.703451 103) (width 0.2) (layer "F.Cu") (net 1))
 (segment (start 143.5 96.4125) (end 141.4875 96.4125) (width 0.2) (layer "F.Cu") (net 1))
 (segment (start 146.4125 96.4125) (end 143.5 96.4125) (width 0.2) (layer "F.Cu") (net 1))
 (segment (start 146.5 112.5) (end 146 112.5) (width 0.2) (layer "F.Cu") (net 1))
 (segment (start 147.45 94.55) (end 147.539 94.461) (width 0.2) (layer "F.Cu") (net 1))
 (segment (start 148.5 102) (end 148.5 99) (width 0.2) (layer "F.Cu") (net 1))
 (segment (start 141.5 98.4125) (end 141.5 99) (width 0.2) (layer "F.Cu") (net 1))
 (segment (start 134.547599 103.7506) (end 134.5 103.703001) (width 0.2) (layer "F.Cu") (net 1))
 (segment (start 143 105) (end 145 103) (width 0.2) (layer "F.Cu") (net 1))
 (segment (start 150 103.5) (end 148.5 102) (width 0.2) (layer "F.Cu") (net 1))
 (segment (start 146.5 113.4) (end 146.5 112.5) (width 0.2) (layer "F.Cu") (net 1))
 (segment (start 135.703451 103) (end 135.500001 102.79655) (width 0.2) (layer "F.Cu") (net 1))
 (segment (start 147.45 95.375) (end 146.4125 96.4125) (width 0.2) (layer "F.Cu") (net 1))
 (segment (start 144.4 115.5) (end 146.5 113.4) (width 0.2) (layer "F.Cu") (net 1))
 (segment (start 134.5 103.703001) (end 134.5 102.79655) (width 0.2) (layer "F.Cu") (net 1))
 (segment (start 147.539 94.461) (end 147.539 87.539) (width 0.2) (layer "F.Cu") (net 1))
 (segment (start 147.45 95.375) (end 147.45 94.55) (width 0.2) (layer "F.Cu") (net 1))
 (segment (start 143.5 96.4125) (end 141.5 98.4125) (width 0.2) (layer "F.Cu") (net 1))
 (segment (start 135.04 87.5) (end 133.65 88.89) (width 0.2) (layer "F.Cu") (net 1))
 (segment (start 144 110.5) (end 143 109.5) (width 0.2) (layer "F.Cu") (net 1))
 (segment (start 147.5 87.5) (end 135.04 87.5) (width 0.2) (layer "F.Cu") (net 1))
 (segment (start 148.5 99) (end 148.5 96.425) (width 0.2) (layer "F.Cu") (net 1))
 (segment (start 143 109.5) (end 143 105) (width 0.2) (layer "F.Cu") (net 1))
 (segment (start 146 112.5) (end 144 110.5) (width 0.2) (layer "F.Cu") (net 1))
 (segment (start 148.5 96.425) (end 147.45 95.375) (width 0.2) (layer "F.Cu") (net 1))
 (segment (start 135.500001 102.79655) (end 135.500001 103.702998) (width 0.2) (layer "F.Cu") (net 1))
 (segment (start 147.539 87.539) (end 147.5 87.5) (width 0.2) (layer "F.Cu") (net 1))
 (segment (start 135.452399 103.7506) (end 134.547599 103.7506) (width 0.2) (layer "F.Cu") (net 1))
 (segment (start 150 104) (end 150 103.5) (width 0.2) (layer "F.Cu") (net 1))
 (segment (start 141.4875 96.4125) (end 140.45 95.375) (width 0.2) (layer "F.Cu") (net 1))
 (segment (start 135.500001 103.702998) (end 135.452399 103.7506) (width 0.2) (layer "F.Cu") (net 1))
 (segment (start 147 117.5) (end 149 115.5) (width 0.2) (layer "F.Cu") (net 9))
 (segment (start 136.921314 108.515965) (end 135.608799 107.20345) (width 0.2) (layer "F.Cu") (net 9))
 (segment (start 151.5 113) (end 151.5 112.5) (width 0.2) (layer "F.Cu") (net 9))
 (segment (start 149 115.5) (end 151.5 113) (width 0.2) (layer "F.Cu") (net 9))
 (segment (start 135.608799 107.20345) (end 135.500001 107.20345) (width 0.2) (layer "F.Cu") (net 9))
 (segment (start 139.04 114.04) (end 142.5 117.5) (width 0.2) (layer "F.Cu") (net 9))
 (segment (start 136.73 114.04) (end 139.04 114.04) (width 0.2) (layer "F.Cu") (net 9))
 (segment (start 136.73 114.04) (end 136.921314 113.848686) (width 0.2) (layer "F.Cu") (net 9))
 (segment (start 136.921314 113.848686) (end 136.921314 108.515965) (width 0.2) (layer "F.Cu") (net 9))
 (segment (start 142.5 117.5) (end 147 117.5) (width 0.2) (layer "F.Cu") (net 9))
 (segment (start 132.25 97.4) (end 130.7 95.85) (width 0.2) (layer "F.Cu") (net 11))
 (segment (start 131.74 83.18) (end 143.81 71.11) (width 0.2) (layer "F.Cu") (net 11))
 (segment (start 130.7 95.85) (end 130.7 90.717006) (width 0.2) (layer "F.Cu") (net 11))
 (segment (start 130.7 90.717006) (end 131.74 89.677006) (width 0.2) (layer "F.Cu") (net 11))
 (segment (start 131.74 89.677006) (end 131.74 83.18) (width 0.2) (layer "F.Cu") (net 11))
 (segment (start 136.19 90.96) (end 136.19 88.89) (width 0.2) (layer "F.Cu") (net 10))
 (segment (start 132.25 94.9) (end 136.19 90.96) (width 0.2) (layer "F.Cu") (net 10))
 (segment (start 134.0476 99.405156) (end 136.452756 97) (width 0.2) (layer "F.Cu") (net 3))
 (segment (start 138.627756 97) (end 139.200001 96.427755) (width 0.2) (layer "F.Cu") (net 3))
 (segment (start 136.452756 97) (end 138.627756 97) (width 0.2) (layer "F.Cu") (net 3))
 (segment (start 139.200001 93.799999) (end 139.5 93.5) (width 0.2) (layer "F.Cu") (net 3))
 (segment (start 139.200001 96.427755) (end 139.200001 93.799999) (width 0.2) (layer "F.Cu") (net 3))
 (segment (start 139.5 93.5) (end 139.5 90.66) (width 0.2) (layer "F.Cu") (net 3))
 (segment (start 139.5 90.66) (end 141.27 88.89) (width 0.2) (layer "F.Cu") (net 3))
 (segment (start 140.946948 93.5) (end 146.5 93.5) (width 0.2) (layer "F.Cu") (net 2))
 (segment (start 146.5 91.58) (end 143.81 88.89) (width 0.2) (layer "F.Cu") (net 2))
 (segment (start 139.85 94.596948) (end 140.946948 93.5) (width 0.2) (layer "F.Cu") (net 2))
 (segment (start 139.85 99.65) (end 139.85 94.596948) (width 0.2) (layer "F.Cu") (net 2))
 (segment (start 135.890101 101) (end 138.5 101) (width 0.2) (layer "F.Cu") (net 2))
 (segment (start 134.999999 102.79655) (end 134.999999 101.890102) (width 0.2) (layer "F.Cu") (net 2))
 (segment (start 134.999999 101.890102) (end 135.890101 101) (width 0.2) (layer "F.Cu") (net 2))
 (segment (start 146.5 93.5) (end 146.5 91.58) (width 0.2) (layer "F.Cu") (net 2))
 (segment (start 138.5 101) (end 139.85 99.65) (width 0.2) (layer "F.Cu") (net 2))
 (segment (start 149 110.5) (end 146.5 110.5) (width 0.2) (layer "F.Cu") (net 14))
 (segment (start 131.65 109.053449) (end 133.499999 107.20345) (width 0.2) (layer "F.Cu") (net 5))
 (segment (start 131.65 114.04) (end 131.65 109.053449) (width 0.2) (layer "F.Cu") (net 5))
 (segment (start 134.999999 107.20345) (end 134.999999 108.13345) (width 0.2) (layer "F.Cu") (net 8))
 (segment (start 136.512655 108.83745) (end 136.512655 109.01345) (width 0.2) (layer "F.Cu") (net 8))
 (segment (start 134.999999 109.71745) (end 134.999999 109.89345) (width 0.2) (layer "F.Cu") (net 8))
 (segment (start 134.999999 109.89345) (end 134.999999 110) (width 0.2) (layer "F.Cu") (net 8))
 (segment (start 135.351999 108.48545) (end 136.160655 108.48545) (width 0.2) (layer "F.Cu") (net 8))
 (segment (start 135.46 110.460001) (end 135.46 111.5) (width 0.2) (layer "F.Cu") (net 8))
 (segment (start 136.160655 109.36545) (end 135.351999 109.36545) (width 0.2) (layer "F.Cu") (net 8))
 (segment (start 134.999999 110) (end 135.46 110.460001) (width 0.2) (layer "F.Cu") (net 8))
 (arc (start 134.999999 108.13345) (mid 135.103097 108.382352) (end 135.351999 108.48545) (width 0.2) (layer "F.Cu") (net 8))
 (arc (start 135.351999 109.36545) (mid 135.103097 109.468548) (end 134.999999 109.71745) (width 0.2) (layer "F.Cu") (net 8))
 (arc (start 136.512655 109.01345) (mid 136.409557 109.262352) (end 136.160655 109.36545) (width 0.2) (layer "F.Cu") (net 8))
 (arc (start 136.160655 108.48545) (mid 136.409557 108.588548) (end 136.512655 108.83745) (width 0.2) (layer "F.Cu") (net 8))
 (segment (start 132.364452 109.697864) (end 132.364452 109.577864) (width 0.2) (layer "F.Cu") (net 6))
 (segment (start 134.000001 107.601978) (end 134.000001 107.20345) (width 0.2) (layer "F.Cu") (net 6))
 (segment (start 133.760001 109.937864) (end 132.604452 109.937864) (width 0.2) (layer "F.Cu") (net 6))
 (segment (start 134.000001 110.419999) (end 134.000001 110.177864) (width 0.2) (layer "F.Cu") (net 6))
 (segment (start 132.92 111.5) (end 134.000001 110.419999) (width 0.2) (layer "F.Cu") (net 6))
 (segment (start 134.000001 109.097864) (end 134.000001 108.977864) (width 0.2) (layer "F.Cu") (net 6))
 (segment (start 132.604452 109.337864) (end 133.760001 109.337864) (width 0.2) (layer "F.Cu") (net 6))
 (segment (start 134.000001 108.977864) (end 134.000001 107.601978) (width 0.2) (layer "F.Cu") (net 6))
 (arc (start 134.000001 110.177864) (mid 133.929707 110.008158) (end 133.760001 109.937864) (width 0.2) (layer "F.Cu") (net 6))
 (arc (start 132.364452 109.577864) (mid 132.434746 109.408158) (end 132.604452 109.337864) (width 0.2) (layer "F.Cu") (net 6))
 (arc (start 133.760001 109.337864) (mid 133.929707 109.26757) (end 134.000001 109.097864) (width 0.2) (layer "F.Cu") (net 6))
 (arc (start 132.604452 109.937864) (mid 132.434746 109.86757) (end 132.364452 109.697864) (width 0.2) (layer "F.Cu") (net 6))
 (segment (start 134.400001 108.599999) (end 134.5 108.5) (width 0.2) (layer "F.Cu") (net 7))
 (segment (start 134.19 114.04) (end 134.400001 113.829999) (width 0.2) (layer "F.Cu") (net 7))
 (segment (start 134.5 108.5) (end 134.5 107.20345) (width 0.2) (layer "F.Cu") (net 7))
 (segment (start 134.400001 113.829999) (end 134.400001 108.599999) (width 0.2) (layer "F.Cu") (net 7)))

